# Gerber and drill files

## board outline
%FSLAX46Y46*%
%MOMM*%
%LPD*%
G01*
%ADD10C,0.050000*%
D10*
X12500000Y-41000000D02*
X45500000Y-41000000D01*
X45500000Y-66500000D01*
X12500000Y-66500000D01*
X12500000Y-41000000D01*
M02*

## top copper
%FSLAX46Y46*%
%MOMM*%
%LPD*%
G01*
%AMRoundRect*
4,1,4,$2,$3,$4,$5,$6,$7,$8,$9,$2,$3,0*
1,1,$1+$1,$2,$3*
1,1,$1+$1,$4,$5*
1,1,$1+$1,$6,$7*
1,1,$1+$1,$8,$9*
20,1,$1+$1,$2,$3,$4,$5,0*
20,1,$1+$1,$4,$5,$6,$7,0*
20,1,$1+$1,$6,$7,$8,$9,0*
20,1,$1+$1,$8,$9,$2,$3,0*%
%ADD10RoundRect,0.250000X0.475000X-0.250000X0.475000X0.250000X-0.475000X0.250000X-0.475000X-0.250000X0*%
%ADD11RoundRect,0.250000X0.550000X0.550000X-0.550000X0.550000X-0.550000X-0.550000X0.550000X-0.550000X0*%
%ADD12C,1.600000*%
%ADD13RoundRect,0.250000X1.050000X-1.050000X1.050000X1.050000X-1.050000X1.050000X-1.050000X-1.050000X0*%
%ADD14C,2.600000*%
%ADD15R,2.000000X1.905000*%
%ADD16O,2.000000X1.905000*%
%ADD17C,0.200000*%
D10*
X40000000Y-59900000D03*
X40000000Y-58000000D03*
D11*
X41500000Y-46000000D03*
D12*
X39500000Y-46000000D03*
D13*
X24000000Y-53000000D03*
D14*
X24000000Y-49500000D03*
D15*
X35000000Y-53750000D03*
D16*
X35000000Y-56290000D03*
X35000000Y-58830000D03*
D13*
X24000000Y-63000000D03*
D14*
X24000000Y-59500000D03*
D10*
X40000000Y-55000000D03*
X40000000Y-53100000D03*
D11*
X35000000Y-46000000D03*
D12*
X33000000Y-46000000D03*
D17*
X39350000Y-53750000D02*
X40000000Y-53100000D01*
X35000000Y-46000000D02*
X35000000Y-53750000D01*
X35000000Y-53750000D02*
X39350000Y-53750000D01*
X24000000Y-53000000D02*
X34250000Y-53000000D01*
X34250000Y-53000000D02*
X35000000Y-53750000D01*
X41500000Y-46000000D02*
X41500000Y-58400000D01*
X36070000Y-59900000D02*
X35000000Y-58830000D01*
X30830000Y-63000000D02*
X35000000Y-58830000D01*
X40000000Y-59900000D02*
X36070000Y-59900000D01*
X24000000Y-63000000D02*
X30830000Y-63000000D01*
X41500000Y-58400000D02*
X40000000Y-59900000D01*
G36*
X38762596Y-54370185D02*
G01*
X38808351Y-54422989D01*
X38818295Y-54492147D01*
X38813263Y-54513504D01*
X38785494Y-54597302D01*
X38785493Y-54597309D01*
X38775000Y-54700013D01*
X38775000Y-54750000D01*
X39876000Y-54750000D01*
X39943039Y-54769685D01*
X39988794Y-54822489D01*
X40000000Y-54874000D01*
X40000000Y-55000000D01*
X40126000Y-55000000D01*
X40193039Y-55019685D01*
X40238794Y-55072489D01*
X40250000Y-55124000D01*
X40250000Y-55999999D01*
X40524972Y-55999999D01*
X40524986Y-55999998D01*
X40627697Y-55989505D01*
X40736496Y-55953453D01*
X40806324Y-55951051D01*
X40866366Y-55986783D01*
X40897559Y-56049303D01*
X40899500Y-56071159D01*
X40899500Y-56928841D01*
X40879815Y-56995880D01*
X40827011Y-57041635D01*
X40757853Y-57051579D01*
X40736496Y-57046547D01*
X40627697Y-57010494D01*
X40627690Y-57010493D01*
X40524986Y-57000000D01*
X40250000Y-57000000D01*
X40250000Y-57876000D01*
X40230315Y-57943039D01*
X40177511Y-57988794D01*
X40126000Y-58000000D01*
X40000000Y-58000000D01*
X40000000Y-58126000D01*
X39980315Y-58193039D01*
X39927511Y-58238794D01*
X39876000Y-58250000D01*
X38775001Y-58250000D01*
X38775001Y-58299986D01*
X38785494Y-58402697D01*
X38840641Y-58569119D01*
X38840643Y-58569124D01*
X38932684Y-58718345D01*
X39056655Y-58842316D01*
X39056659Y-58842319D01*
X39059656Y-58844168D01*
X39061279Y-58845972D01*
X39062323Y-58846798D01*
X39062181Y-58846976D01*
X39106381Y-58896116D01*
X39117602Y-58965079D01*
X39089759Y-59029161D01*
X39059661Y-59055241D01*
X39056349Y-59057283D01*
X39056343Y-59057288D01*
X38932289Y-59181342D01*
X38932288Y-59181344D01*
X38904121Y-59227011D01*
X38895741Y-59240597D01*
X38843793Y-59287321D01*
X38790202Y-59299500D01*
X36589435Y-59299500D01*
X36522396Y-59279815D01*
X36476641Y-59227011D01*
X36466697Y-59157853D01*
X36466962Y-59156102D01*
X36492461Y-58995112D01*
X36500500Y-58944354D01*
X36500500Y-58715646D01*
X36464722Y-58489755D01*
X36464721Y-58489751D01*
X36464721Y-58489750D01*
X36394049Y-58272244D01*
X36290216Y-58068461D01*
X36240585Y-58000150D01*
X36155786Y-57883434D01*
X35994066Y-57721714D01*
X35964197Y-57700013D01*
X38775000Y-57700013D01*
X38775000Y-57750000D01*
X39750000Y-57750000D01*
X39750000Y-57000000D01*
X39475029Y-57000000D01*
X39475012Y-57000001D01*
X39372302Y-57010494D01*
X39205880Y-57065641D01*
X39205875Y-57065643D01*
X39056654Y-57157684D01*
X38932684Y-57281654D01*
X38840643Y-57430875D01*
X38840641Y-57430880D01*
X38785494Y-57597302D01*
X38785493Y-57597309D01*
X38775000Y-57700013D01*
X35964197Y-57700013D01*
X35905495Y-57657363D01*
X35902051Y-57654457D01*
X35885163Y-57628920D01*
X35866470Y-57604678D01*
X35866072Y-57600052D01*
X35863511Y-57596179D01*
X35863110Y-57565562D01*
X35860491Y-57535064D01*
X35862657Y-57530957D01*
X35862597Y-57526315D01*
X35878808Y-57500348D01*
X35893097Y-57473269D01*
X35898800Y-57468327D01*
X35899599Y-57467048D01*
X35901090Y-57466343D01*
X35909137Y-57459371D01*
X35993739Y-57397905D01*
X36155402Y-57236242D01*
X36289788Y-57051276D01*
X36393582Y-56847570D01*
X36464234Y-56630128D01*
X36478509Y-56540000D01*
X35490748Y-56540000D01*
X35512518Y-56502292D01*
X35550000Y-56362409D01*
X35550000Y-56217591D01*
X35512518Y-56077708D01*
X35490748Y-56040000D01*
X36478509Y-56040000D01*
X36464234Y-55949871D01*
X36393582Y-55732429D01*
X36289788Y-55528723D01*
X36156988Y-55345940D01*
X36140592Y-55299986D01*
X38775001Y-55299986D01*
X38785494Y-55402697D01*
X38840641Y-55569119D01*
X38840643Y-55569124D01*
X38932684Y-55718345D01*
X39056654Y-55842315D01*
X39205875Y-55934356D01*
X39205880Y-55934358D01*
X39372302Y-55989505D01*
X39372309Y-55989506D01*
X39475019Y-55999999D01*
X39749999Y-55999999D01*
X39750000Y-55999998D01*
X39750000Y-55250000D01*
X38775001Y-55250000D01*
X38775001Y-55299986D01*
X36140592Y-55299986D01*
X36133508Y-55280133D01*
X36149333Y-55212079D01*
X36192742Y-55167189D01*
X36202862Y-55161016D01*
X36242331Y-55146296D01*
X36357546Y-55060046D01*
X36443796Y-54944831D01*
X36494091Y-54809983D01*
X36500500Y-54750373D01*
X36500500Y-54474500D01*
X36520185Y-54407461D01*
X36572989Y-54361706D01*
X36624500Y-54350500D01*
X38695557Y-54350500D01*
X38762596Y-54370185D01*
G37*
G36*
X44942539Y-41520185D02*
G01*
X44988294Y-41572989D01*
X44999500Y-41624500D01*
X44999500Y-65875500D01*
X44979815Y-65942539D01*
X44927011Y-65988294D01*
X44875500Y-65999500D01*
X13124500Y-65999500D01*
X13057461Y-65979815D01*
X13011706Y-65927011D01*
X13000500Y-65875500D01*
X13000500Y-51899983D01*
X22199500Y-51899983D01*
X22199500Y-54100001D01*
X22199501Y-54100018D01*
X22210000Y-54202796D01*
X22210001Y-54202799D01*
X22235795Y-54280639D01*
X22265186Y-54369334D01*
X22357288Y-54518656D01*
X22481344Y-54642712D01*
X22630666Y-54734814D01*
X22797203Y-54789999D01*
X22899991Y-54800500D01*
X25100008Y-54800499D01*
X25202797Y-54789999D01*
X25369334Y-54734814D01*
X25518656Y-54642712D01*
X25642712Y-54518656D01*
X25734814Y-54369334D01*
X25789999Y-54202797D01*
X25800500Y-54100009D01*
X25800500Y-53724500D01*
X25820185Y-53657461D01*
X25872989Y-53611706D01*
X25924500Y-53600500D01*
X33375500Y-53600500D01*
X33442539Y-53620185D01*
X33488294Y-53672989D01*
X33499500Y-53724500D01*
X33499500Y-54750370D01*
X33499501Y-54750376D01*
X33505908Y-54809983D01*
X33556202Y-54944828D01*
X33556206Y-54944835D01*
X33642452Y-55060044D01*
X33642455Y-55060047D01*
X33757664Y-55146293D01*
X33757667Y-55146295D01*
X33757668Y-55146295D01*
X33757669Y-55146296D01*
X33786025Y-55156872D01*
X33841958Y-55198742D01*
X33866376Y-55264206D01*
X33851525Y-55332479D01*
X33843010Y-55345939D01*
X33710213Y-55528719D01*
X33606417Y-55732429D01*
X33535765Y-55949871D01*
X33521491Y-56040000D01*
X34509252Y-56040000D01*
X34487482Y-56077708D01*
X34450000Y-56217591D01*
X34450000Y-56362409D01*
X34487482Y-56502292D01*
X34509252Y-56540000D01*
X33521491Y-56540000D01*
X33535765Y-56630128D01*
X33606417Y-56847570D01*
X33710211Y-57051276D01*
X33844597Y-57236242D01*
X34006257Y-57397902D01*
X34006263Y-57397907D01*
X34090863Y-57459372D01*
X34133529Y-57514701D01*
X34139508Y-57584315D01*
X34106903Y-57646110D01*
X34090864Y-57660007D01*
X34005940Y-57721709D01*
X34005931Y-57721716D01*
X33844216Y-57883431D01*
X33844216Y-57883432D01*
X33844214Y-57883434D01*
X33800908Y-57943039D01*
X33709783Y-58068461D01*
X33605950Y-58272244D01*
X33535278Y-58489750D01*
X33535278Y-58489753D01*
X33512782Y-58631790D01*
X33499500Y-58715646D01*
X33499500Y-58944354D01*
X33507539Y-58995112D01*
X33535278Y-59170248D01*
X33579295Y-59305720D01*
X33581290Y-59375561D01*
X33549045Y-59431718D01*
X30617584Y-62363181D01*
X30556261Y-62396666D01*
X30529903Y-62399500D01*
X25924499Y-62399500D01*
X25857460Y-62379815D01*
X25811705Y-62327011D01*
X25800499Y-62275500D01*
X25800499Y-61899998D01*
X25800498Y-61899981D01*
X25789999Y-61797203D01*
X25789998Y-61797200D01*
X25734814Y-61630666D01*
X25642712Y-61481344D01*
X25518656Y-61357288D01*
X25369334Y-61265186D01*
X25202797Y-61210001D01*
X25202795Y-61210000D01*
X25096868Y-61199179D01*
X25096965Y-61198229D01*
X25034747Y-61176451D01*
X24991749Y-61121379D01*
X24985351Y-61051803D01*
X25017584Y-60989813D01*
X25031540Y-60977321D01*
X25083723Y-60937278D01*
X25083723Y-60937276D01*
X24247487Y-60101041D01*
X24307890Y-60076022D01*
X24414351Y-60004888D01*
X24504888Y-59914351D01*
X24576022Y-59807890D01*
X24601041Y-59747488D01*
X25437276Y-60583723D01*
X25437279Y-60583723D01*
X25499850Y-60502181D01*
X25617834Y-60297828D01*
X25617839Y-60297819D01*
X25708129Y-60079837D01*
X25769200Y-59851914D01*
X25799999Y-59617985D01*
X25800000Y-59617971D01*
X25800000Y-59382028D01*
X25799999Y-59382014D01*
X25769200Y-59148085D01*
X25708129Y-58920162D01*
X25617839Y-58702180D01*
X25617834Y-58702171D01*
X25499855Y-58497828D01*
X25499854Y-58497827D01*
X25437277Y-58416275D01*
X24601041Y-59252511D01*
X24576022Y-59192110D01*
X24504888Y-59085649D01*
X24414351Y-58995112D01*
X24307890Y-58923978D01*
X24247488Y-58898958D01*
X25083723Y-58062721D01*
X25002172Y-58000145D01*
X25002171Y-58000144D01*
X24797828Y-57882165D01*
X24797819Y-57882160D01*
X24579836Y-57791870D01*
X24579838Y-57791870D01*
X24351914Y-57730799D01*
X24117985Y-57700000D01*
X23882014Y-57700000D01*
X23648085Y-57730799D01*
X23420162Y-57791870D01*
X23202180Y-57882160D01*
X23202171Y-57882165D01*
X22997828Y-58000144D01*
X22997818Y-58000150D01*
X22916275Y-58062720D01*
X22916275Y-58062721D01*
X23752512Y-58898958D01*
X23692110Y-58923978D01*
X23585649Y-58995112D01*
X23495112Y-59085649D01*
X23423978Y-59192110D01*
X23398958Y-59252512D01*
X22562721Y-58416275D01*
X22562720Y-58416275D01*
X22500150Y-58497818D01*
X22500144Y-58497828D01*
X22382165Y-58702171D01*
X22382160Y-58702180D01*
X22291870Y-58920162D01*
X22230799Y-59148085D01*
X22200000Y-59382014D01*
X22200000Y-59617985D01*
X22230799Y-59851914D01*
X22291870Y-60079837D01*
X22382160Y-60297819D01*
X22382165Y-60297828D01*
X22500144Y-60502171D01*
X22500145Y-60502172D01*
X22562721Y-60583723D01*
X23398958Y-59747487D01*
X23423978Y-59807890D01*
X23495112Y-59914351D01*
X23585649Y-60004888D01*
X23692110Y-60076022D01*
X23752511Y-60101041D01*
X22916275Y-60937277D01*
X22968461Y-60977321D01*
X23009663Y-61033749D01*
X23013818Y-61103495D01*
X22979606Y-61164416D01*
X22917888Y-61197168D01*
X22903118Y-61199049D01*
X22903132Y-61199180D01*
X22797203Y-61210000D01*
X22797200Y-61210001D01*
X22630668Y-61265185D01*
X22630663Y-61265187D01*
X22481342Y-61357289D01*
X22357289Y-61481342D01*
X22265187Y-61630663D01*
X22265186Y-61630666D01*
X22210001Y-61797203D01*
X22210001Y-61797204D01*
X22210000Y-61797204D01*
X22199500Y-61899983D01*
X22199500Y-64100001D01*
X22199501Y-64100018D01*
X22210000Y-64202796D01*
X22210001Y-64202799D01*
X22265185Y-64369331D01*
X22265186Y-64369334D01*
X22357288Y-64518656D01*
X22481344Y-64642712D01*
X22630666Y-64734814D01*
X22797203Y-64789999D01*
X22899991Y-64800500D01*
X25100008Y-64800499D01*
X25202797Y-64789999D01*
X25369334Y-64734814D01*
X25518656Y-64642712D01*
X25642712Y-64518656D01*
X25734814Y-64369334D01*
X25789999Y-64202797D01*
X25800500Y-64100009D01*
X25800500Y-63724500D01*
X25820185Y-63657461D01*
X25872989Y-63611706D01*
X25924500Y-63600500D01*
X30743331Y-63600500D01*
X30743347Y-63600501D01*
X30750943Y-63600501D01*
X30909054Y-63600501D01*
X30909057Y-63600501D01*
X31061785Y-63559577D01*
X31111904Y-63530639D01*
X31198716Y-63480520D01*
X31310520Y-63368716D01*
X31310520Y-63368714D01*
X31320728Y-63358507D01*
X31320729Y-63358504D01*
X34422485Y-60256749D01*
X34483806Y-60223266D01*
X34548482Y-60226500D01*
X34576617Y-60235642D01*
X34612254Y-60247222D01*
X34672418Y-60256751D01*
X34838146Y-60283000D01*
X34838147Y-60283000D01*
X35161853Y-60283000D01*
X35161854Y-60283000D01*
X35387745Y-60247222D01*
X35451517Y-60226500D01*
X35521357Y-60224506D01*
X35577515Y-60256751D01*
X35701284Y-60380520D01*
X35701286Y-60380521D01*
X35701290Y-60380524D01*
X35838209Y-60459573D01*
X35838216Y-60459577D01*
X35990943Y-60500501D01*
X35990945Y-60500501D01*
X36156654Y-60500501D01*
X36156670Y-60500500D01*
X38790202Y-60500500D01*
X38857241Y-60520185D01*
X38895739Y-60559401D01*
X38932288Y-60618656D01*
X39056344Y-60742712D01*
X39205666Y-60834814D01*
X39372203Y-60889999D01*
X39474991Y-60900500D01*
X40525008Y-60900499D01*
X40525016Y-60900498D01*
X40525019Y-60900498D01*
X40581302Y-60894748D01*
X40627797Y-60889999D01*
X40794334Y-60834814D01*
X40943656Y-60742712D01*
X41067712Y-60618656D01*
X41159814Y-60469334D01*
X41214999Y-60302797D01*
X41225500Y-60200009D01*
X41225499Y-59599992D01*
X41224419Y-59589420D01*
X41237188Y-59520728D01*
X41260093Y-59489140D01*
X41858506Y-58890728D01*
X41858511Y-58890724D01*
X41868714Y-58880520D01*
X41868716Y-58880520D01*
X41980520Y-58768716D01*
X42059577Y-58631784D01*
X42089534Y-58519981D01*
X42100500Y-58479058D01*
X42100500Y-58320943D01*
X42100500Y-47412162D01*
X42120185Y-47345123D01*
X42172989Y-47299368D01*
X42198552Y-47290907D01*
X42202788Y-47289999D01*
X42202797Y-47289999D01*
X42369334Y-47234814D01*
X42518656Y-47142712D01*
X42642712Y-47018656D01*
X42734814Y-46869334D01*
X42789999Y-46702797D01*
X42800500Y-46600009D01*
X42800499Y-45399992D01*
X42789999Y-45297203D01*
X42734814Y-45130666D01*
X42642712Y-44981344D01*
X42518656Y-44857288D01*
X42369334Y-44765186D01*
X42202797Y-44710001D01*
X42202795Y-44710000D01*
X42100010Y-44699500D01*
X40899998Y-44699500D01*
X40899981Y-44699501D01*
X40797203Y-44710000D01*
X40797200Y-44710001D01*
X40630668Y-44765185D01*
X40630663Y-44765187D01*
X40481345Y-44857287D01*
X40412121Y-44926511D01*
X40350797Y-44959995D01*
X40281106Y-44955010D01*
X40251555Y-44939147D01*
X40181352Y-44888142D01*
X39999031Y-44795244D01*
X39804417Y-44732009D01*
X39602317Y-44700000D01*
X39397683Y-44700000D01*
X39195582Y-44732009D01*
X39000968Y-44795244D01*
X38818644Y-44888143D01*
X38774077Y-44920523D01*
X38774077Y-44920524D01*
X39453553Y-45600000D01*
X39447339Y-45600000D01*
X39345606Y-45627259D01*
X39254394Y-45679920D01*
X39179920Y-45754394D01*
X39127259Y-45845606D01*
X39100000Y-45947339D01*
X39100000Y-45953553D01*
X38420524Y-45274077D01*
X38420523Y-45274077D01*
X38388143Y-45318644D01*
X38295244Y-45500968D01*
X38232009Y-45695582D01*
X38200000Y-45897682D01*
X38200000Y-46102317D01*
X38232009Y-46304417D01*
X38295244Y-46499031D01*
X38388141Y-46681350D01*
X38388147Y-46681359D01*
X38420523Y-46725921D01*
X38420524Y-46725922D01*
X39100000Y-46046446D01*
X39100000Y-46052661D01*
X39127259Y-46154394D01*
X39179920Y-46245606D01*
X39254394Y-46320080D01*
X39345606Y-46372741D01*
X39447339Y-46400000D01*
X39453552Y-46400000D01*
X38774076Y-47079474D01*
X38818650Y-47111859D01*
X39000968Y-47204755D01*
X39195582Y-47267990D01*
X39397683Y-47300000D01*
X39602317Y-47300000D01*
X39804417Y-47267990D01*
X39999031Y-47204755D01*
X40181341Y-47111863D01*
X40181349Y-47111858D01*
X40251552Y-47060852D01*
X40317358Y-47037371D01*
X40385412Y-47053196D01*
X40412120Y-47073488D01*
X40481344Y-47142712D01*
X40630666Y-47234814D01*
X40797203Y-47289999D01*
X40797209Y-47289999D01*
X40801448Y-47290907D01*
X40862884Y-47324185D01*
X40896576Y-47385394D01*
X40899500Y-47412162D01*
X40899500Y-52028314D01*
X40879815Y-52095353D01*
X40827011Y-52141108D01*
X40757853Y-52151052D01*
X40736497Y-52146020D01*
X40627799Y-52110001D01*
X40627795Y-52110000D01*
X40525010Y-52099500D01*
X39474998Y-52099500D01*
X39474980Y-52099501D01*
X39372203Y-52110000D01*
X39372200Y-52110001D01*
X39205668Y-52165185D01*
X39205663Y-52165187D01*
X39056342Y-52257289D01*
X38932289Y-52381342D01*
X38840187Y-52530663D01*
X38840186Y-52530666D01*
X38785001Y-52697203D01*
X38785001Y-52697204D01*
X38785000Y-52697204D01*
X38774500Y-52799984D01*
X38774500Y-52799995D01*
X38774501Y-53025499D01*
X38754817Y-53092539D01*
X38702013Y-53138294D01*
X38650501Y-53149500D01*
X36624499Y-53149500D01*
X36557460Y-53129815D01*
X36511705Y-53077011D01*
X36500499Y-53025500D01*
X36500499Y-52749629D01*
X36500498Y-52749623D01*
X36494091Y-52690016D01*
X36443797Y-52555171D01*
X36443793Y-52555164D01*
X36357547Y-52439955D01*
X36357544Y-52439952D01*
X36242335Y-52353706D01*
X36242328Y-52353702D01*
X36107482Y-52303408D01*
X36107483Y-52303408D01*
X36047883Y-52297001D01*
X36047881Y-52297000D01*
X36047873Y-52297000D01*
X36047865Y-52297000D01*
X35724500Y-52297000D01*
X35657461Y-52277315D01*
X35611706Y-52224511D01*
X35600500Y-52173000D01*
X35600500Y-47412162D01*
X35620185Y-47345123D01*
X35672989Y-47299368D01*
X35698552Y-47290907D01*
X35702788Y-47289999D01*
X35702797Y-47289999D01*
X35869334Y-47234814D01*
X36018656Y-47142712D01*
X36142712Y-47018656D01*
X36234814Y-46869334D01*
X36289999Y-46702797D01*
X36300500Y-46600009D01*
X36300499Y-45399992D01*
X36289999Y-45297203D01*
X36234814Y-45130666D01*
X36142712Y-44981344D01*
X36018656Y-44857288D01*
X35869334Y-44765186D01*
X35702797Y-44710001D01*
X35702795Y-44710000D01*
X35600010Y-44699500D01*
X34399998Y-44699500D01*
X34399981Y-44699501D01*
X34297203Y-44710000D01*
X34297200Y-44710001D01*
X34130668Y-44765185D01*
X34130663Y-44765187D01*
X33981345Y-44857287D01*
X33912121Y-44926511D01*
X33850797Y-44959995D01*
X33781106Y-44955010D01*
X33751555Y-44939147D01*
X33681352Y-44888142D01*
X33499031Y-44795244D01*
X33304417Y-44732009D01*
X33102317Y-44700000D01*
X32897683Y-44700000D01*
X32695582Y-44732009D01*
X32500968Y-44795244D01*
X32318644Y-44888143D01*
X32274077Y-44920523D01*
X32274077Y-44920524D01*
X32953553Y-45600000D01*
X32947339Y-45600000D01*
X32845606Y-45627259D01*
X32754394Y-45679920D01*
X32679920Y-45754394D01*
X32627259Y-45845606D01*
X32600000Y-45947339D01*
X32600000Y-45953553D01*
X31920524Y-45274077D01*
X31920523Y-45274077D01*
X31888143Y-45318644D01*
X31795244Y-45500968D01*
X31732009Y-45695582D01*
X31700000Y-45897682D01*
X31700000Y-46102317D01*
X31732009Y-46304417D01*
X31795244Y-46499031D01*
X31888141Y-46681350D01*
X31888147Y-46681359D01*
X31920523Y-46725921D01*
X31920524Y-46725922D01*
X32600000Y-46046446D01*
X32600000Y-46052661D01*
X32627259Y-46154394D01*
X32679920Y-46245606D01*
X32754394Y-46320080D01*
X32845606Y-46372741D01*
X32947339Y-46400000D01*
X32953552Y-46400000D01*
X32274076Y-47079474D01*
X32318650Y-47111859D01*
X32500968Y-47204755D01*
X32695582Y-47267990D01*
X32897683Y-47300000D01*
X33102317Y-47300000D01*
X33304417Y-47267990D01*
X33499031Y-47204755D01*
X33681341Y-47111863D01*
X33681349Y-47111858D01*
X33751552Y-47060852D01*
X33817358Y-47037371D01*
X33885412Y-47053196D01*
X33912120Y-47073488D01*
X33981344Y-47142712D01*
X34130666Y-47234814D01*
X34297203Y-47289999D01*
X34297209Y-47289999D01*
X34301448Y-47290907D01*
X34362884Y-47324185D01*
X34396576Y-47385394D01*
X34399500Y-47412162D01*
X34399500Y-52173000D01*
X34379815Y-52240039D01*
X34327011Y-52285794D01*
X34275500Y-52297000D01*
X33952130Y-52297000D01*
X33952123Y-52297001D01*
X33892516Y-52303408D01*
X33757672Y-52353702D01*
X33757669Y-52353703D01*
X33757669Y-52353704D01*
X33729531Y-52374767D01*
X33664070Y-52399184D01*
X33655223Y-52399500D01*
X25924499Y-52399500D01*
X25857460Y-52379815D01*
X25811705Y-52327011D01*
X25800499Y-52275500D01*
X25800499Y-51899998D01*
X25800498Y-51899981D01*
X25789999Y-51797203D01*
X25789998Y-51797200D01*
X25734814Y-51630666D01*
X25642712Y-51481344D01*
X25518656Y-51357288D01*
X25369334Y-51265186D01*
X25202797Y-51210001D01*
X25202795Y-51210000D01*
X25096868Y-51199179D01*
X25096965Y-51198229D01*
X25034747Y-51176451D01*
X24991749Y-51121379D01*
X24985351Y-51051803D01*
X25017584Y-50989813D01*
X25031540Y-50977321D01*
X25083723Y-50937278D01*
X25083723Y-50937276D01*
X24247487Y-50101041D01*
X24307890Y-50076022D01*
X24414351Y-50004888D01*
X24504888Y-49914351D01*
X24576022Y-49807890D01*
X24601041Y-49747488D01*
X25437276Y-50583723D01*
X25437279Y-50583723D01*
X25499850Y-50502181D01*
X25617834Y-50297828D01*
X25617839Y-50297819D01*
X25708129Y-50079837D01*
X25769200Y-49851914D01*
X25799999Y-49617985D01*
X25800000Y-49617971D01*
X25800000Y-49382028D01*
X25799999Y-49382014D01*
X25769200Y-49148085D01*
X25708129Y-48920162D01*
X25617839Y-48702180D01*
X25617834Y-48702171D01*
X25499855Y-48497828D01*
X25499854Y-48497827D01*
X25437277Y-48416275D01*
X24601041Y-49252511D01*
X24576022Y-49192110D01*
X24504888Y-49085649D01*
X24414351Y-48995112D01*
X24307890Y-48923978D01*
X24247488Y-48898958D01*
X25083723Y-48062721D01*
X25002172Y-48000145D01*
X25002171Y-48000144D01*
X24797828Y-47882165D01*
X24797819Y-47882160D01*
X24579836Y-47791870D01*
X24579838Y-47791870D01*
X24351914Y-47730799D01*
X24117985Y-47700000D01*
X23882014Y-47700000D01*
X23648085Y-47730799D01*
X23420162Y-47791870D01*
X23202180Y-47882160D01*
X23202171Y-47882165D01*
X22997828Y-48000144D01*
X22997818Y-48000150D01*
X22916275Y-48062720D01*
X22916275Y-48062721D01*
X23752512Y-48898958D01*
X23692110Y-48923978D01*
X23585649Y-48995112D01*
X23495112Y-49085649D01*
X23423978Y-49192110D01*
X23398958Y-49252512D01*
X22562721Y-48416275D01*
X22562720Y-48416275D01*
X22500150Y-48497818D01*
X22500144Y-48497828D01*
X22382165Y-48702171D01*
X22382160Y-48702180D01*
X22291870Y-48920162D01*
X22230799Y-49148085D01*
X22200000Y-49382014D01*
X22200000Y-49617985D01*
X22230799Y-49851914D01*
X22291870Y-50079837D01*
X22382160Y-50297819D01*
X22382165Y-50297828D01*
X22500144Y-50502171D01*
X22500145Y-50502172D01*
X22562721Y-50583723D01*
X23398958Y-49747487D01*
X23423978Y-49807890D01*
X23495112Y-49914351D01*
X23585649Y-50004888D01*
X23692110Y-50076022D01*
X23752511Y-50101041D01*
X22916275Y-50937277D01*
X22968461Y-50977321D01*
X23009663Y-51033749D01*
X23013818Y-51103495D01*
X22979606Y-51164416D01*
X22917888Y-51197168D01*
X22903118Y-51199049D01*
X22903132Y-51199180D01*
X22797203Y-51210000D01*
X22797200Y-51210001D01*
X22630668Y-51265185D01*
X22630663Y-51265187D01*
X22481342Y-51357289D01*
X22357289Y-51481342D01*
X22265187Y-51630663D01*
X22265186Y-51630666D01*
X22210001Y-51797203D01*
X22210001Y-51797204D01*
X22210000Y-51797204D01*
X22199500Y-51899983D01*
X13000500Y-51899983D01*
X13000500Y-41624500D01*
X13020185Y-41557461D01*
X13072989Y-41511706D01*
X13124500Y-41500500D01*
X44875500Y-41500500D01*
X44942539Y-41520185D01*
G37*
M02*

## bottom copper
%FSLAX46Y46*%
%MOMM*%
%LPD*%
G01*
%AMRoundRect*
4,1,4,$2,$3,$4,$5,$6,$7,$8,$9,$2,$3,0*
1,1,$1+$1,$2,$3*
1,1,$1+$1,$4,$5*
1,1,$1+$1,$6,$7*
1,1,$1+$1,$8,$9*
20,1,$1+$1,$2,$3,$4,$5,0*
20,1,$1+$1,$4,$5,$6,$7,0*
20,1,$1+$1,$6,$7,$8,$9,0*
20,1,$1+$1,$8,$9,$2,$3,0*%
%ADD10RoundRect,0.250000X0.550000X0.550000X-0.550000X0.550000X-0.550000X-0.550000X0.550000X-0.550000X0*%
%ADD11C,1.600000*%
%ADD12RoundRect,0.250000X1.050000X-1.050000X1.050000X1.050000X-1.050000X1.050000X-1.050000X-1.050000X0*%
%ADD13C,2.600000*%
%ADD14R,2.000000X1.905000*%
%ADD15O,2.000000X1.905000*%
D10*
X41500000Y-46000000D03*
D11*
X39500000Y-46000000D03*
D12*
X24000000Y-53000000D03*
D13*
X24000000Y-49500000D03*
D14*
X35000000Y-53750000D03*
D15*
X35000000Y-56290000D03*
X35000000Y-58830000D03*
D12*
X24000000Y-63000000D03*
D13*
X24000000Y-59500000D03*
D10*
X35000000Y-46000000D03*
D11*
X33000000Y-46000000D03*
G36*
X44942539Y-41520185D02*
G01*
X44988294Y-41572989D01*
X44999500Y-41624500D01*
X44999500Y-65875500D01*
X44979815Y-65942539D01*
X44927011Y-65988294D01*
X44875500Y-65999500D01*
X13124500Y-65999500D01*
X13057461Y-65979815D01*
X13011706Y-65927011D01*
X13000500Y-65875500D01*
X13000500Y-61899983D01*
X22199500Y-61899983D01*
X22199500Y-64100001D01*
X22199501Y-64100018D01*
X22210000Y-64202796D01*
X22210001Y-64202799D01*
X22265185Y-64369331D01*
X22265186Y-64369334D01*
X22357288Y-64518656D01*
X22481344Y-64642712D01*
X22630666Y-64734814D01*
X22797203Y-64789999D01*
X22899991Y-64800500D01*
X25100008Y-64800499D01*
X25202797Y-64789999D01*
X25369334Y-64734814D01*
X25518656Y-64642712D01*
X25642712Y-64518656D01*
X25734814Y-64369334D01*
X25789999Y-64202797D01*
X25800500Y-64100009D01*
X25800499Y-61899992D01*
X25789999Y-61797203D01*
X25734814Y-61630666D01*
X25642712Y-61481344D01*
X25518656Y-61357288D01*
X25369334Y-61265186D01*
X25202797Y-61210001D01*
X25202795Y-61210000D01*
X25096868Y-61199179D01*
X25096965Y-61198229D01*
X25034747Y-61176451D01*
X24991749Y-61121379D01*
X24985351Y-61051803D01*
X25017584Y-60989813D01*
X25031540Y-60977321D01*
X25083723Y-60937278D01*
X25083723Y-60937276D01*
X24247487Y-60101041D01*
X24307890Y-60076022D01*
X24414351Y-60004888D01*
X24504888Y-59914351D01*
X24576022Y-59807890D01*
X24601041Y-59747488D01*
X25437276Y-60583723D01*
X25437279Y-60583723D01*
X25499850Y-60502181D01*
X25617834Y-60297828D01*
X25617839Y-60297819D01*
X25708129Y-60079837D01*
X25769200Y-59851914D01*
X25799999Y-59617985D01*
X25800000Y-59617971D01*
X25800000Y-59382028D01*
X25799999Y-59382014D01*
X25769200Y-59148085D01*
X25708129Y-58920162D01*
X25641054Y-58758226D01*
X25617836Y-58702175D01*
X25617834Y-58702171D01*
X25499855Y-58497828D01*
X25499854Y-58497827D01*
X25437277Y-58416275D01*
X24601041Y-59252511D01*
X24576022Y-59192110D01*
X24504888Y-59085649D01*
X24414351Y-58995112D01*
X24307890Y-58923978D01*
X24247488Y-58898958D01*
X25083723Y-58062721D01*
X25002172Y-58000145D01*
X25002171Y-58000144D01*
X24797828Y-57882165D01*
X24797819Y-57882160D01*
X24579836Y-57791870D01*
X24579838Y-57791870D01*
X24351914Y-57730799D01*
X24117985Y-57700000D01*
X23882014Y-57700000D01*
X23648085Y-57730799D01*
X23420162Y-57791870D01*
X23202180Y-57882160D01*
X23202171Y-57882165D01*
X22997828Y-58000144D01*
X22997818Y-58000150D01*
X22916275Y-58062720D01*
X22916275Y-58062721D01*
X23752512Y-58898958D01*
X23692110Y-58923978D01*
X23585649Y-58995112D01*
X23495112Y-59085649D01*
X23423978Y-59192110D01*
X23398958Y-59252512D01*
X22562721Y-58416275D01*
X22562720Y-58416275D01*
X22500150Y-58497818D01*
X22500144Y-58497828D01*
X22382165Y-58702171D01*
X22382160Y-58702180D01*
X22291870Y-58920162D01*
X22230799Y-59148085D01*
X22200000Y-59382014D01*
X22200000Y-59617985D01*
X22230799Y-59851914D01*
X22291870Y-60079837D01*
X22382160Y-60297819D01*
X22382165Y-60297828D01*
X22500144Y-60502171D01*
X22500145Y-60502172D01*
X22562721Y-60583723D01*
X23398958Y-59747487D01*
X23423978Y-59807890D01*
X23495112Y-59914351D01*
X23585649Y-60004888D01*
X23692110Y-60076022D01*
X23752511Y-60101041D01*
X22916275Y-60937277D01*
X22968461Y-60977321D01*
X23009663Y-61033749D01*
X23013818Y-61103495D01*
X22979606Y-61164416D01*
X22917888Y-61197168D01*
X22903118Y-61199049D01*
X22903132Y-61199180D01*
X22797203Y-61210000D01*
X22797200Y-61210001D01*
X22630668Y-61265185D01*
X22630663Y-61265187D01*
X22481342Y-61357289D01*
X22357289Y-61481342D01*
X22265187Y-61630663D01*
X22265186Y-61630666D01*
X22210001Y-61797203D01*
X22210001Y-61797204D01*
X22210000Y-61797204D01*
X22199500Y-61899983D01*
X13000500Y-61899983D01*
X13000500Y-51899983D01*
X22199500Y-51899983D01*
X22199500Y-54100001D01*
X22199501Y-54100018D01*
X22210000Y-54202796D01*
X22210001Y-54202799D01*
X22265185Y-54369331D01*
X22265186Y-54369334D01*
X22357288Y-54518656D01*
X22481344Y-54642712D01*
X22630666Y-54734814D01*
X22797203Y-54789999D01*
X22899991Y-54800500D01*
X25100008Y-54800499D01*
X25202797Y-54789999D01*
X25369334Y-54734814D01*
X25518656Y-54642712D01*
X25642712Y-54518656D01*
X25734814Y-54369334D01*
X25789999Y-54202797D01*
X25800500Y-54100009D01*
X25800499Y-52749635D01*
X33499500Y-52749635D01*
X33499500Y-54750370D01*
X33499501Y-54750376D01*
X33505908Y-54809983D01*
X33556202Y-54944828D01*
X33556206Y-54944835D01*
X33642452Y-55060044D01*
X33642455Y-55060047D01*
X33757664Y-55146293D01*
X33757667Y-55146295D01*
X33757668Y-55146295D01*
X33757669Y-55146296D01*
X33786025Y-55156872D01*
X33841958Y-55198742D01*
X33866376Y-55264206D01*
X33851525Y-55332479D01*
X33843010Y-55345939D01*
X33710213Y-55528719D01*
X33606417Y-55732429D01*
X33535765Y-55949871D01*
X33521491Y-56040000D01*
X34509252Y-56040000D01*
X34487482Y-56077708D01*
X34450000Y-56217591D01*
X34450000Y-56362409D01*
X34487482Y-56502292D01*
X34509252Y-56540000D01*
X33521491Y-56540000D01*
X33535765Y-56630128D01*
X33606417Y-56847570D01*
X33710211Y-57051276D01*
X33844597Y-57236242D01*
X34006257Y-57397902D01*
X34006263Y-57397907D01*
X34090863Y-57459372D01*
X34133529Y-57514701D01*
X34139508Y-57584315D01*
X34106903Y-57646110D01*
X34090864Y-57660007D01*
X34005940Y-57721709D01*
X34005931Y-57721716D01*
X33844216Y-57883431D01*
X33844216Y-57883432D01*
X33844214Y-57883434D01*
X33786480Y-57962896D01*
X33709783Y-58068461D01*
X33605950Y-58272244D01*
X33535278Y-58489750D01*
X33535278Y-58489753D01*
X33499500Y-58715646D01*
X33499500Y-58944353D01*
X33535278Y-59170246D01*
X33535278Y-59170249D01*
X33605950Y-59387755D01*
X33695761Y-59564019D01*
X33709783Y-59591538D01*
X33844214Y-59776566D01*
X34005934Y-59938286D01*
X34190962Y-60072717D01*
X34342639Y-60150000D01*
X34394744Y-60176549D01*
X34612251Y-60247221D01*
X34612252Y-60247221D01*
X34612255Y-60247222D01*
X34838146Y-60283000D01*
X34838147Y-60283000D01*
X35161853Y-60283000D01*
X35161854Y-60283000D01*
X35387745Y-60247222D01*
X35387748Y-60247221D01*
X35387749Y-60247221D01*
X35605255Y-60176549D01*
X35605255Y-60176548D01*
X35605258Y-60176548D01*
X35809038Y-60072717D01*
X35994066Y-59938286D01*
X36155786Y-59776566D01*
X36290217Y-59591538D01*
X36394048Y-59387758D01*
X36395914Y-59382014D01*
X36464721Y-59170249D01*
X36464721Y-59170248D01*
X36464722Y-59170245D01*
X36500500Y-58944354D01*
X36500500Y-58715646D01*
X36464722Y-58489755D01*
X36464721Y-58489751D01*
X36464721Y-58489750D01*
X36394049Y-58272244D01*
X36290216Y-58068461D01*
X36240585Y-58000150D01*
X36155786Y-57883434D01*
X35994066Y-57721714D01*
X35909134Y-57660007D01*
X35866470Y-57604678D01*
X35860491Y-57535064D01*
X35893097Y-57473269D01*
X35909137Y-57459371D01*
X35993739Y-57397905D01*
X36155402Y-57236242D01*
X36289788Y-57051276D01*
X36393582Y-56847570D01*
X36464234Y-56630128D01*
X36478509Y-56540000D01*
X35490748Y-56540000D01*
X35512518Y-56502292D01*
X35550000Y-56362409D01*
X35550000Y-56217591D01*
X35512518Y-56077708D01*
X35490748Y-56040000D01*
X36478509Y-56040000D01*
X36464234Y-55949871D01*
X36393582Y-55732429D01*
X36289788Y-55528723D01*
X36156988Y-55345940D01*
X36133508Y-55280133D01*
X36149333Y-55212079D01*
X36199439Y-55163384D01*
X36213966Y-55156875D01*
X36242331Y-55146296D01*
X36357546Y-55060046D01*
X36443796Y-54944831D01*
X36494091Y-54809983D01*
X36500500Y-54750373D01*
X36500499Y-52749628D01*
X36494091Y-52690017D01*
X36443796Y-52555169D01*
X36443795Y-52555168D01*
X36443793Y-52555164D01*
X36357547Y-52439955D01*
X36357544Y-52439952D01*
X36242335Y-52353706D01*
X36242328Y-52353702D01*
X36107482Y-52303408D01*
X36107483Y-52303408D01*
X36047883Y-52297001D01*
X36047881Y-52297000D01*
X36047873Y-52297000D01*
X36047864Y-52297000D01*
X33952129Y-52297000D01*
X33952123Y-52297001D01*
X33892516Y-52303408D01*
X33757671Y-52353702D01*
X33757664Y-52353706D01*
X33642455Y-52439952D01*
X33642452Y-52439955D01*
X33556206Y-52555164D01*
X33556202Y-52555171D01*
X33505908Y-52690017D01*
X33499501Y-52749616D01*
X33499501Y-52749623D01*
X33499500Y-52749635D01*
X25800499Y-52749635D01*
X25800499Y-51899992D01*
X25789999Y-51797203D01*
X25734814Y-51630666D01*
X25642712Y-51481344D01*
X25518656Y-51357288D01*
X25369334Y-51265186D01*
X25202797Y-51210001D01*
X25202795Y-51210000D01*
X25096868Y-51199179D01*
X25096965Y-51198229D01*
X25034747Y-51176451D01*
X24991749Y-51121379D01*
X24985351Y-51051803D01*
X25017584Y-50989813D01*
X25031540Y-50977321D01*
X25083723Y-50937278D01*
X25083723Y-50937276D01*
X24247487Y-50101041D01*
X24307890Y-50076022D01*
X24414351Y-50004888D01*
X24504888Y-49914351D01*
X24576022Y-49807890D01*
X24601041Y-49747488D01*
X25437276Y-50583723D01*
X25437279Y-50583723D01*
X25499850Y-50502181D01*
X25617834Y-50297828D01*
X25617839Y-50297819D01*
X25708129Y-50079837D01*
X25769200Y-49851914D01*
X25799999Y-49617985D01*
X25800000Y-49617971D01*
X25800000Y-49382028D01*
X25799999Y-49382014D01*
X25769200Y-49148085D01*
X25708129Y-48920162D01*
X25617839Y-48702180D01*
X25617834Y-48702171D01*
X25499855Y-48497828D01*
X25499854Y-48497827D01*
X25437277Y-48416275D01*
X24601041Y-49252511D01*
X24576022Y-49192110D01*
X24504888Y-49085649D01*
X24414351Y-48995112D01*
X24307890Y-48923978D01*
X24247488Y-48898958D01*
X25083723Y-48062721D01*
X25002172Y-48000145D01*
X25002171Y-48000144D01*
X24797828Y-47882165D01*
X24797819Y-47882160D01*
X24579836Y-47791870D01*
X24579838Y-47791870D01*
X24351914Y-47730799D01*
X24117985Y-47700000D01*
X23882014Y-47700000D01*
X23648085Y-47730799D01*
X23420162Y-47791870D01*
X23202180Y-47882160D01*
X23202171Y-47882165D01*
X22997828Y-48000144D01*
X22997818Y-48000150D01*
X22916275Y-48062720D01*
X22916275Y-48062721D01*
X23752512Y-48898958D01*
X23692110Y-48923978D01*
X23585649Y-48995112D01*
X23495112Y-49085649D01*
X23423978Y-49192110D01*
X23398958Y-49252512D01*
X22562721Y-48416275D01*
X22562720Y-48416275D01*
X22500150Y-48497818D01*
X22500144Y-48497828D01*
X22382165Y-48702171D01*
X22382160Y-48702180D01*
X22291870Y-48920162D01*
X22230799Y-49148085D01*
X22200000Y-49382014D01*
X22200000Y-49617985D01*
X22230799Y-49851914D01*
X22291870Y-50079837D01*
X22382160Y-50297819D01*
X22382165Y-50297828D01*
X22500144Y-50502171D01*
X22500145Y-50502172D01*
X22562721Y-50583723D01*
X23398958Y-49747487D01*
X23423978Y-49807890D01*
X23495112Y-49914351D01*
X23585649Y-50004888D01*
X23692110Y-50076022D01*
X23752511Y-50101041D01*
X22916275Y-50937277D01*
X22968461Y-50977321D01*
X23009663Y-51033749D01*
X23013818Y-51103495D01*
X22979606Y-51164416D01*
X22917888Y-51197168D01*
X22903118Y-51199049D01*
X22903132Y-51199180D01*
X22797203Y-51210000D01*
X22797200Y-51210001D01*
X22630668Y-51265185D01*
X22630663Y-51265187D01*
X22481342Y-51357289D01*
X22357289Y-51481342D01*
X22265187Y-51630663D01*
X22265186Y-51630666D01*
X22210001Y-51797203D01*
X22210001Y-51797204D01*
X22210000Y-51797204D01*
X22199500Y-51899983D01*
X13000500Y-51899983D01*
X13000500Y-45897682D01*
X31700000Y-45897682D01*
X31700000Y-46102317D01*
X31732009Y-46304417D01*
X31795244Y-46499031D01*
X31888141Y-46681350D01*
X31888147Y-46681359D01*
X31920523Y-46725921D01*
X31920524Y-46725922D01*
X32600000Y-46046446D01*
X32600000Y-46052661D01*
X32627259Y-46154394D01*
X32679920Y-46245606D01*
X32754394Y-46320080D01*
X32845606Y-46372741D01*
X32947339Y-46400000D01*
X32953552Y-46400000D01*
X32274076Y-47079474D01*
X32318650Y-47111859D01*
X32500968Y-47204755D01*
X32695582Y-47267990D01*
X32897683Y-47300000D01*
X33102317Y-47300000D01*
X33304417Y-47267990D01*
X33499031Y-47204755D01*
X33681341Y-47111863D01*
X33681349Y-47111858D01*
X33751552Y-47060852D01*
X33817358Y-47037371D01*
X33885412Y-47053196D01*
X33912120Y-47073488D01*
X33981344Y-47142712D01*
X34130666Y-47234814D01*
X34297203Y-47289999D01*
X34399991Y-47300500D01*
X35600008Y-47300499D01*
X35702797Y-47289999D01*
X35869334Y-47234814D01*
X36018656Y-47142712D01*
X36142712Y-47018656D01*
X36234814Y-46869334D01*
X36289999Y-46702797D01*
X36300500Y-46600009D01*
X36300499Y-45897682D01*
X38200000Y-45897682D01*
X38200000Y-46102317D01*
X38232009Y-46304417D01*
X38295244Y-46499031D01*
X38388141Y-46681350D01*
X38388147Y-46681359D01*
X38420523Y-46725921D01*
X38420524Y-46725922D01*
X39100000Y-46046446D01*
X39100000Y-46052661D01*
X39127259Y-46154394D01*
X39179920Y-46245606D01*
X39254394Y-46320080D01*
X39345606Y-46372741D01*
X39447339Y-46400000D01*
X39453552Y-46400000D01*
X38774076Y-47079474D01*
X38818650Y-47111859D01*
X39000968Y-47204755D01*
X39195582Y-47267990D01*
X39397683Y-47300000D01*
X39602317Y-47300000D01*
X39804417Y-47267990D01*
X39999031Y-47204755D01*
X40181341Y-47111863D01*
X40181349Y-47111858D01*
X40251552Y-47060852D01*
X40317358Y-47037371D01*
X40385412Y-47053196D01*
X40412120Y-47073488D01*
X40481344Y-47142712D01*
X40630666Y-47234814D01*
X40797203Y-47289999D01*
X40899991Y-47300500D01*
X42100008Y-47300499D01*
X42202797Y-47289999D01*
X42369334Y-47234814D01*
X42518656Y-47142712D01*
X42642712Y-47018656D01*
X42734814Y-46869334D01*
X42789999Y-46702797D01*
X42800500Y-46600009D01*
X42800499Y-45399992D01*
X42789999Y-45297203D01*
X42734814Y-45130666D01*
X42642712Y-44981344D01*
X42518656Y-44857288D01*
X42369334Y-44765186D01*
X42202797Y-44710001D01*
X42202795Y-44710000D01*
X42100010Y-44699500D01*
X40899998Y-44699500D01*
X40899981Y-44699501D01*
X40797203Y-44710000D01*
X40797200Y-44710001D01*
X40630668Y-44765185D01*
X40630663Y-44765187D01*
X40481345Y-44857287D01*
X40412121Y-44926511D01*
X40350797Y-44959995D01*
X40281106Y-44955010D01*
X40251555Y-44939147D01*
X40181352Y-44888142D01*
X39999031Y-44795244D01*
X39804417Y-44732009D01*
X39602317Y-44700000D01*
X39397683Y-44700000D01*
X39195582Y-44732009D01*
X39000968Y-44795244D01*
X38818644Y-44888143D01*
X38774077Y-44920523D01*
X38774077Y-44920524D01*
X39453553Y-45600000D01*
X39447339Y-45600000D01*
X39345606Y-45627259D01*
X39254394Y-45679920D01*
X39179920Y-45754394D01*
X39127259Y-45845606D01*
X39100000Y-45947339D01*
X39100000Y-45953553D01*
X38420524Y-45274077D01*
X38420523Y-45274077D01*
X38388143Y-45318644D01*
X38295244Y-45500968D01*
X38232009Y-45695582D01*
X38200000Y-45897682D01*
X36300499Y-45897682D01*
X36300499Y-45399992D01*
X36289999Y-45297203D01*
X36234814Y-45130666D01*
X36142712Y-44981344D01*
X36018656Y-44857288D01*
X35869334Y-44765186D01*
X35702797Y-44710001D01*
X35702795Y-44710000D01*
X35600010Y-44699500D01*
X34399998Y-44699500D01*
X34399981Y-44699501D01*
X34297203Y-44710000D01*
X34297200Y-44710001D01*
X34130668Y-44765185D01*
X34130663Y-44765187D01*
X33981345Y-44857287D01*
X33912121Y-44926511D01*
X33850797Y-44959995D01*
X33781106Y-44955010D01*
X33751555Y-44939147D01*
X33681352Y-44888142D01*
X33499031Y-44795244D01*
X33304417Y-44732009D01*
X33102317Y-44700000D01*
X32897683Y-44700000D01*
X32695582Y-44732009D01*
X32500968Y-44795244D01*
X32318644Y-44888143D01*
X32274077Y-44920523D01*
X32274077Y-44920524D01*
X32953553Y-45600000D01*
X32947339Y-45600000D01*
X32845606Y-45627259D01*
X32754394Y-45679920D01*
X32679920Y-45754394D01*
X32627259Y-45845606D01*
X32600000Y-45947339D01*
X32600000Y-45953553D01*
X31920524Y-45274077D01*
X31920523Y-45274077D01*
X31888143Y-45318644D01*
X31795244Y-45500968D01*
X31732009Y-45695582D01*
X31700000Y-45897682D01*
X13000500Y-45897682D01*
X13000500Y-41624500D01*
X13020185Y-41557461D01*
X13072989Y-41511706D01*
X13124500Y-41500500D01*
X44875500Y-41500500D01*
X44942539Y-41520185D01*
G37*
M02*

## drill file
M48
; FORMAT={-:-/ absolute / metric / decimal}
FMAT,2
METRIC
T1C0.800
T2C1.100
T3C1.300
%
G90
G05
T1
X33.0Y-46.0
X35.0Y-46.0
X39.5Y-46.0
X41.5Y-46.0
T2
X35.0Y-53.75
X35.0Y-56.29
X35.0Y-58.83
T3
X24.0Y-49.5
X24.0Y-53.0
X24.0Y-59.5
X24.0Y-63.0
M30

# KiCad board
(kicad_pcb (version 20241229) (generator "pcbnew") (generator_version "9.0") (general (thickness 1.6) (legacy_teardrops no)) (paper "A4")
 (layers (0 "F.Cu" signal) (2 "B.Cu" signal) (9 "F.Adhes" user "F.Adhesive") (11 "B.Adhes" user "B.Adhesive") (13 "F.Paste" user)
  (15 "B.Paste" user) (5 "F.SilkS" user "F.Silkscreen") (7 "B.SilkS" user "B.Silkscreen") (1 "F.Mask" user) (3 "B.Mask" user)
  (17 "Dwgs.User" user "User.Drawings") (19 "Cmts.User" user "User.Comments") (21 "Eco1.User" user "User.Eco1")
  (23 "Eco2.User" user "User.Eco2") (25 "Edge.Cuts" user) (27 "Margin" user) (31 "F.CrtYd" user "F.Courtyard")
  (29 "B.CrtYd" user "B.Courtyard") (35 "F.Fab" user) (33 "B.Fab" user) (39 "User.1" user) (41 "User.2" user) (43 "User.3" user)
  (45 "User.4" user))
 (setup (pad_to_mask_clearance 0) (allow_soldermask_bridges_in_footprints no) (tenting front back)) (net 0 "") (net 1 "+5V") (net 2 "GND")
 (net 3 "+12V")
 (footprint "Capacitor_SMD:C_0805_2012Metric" (layer "F.Cu") (at 40 58.95 90)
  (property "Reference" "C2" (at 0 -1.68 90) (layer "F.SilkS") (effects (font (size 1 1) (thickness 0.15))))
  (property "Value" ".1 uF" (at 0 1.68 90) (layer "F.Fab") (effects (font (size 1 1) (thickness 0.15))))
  (pad "1" smd roundrect (at -0.95 0 90) (size 1 1.45) (layers "F.Cu" "F.Mask" "F.Paste") (roundrect_rratio 0.25) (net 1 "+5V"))
  (pad "2" smd roundrect (at 0.95 0 90) (size 1 1.45) (layers "F.Cu" "F.Mask" "F.Paste") (roundrect_rratio 0.25) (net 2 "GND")))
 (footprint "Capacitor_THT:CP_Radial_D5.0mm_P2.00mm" (layer "F.Cu") (at 41.5 46 180)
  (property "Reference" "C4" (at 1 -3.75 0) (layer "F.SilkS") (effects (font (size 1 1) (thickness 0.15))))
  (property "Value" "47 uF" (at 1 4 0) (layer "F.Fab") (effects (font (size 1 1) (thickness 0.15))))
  (pad "1" thru_hole roundrect (at 0 0 180) (size 1.6 1.6) (drill 0.8) (layers "*.Cu" "*.Mask") (remove_unused_layers no)
   (roundrect_rratio 0.15625) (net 1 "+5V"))
  (pad "2" thru_hole circle (at 2 0 180) (size 1.6 1.6) (drill 0.8) (layers "*.Cu" "*.Mask") (remove_unused_layers no) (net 2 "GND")))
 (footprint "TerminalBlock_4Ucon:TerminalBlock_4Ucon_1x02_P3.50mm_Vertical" (layer "F.Cu") (at 24 53 90)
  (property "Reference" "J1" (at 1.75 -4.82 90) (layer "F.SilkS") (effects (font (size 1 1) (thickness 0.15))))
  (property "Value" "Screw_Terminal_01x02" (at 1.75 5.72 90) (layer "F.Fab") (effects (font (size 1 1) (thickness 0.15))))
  (pad "1" thru_hole roundrect (at 0 0 90) (size 2.6 2.6) (drill 1.3) (layers "*.Cu" "*.Mask") (remove_unused_layers no)
   (roundrect_rratio 0.096154) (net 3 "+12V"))
  (pad "2" thru_hole circle (at 3.5 0 90) (size 2.6 2.6) (drill 1.3) (layers "*.Cu" "*.Mask") (remove_unused_layers no) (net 2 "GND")))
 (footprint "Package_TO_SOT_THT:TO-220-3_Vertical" (layer "F.Cu") (at 35 53.75 -90)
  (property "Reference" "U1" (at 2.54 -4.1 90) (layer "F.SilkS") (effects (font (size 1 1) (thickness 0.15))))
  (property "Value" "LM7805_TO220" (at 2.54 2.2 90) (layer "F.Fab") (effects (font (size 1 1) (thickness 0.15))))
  (pad "1" thru_hole rect (at 0 0 270) (size 1.905 2) (drill 1.1) (layers "*.Cu" "*.Mask") (remove_unused_layers no) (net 3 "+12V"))
  (pad "2" thru_hole oval (at 2.54 0 270) (size 1.905 2) (drill 1.1) (layers "*.Cu" "*.Mask") (remove_unused_layers no) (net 2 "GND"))
  (pad "3" thru_hole oval (at 5.08 0 270) (size 1.905 2) (drill 1.1) (layers "*.Cu" "*.Mask") (remove_unused_layers no) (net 1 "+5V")))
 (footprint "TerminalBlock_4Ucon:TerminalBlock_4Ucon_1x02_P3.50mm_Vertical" (layer "F.Cu") (at 24 63 90)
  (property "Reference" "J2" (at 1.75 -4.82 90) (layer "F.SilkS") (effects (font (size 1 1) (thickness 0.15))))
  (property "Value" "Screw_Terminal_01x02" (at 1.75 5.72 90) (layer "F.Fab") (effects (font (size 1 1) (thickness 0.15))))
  (pad "1" thru_hole roundrect (at 0 0 90) (size 2.6 2.6) (drill 1.3) (layers "*.Cu" "*.Mask") (remove_unused_layers no)
   (roundrect_rratio 0.096154) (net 1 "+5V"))
  (pad "2" thru_hole circle (at 3.5 0 90) (size 2.6 2.6) (drill 1.3) (layers "*.Cu" "*.Mask") (remove_unused_layers no) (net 2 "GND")))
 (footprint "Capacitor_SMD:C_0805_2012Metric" (layer "F.Cu") (at 40 54.05 90)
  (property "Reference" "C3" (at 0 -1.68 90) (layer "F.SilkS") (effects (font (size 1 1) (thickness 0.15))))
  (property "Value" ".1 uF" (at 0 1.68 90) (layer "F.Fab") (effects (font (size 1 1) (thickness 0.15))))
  (pad "1" smd roundrect (at -0.95 0 90) (size 1 1.45) (layers "F.Cu" "F.Mask" "F.Paste") (roundrect_rratio 0.25) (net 2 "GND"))
  (pad "2" smd roundrect (at 0.95 0 90) (size 1 1.45) (layers "F.Cu" "F.Mask" "F.Paste") (roundrect_rratio 0.25) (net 3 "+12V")))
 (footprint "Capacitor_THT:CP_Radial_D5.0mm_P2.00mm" (layer "F.Cu") (at 35 46 180)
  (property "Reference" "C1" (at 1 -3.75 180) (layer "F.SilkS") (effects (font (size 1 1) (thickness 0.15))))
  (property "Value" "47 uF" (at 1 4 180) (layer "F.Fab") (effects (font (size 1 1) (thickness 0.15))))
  (pad "1" thru_hole roundrect (at 0 0 180) (size 1.6 1.6) (drill 0.8) (layers "*.Cu" "*.Mask") (remove_unused_layers no)
   (roundrect_rratio 0.15625) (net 3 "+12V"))
  (pad "2" thru_hole circle (at 2 0 180) (size 1.6 1.6) (drill 0.8) (layers "*.Cu" "*.Mask") (remove_unused_layers no) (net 2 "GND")))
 (gr_rect (start 12.5 41) (end 45.5 66.5) (stroke (width 0.05) (type default)) (fill no) (layer "Edge.Cuts"))
 (segment (start 39.35 53.75) (end 40 53.1) (width 0.2) (layer "F.Cu") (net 3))
 (segment (start 35 46) (end 35 53.75) (width 0.2) (layer "F.Cu") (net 3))
 (segment (start 35 53.75) (end 39.35 53.75) (width 0.2) (layer "F.Cu") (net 3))
 (segment (start 24 53) (end 34.25 53) (width 0.2) (layer "F.Cu") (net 3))
 (segment (start 34.25 53) (end 35 53.75) (width 0.2) (layer "F.Cu") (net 3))
 (segment (start 41.5 46) (end 41.5 58.4) (width 0.2) (layer "F.Cu") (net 1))
 (segment (start 36.07 59.9) (end 35 58.83) (width 0.2) (layer "F.Cu") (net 1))
 (segment (start 30.83 63) (end 35 58.83) (width 0.2) (layer "F.Cu") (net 1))
 (segment (start 40 59.9) (end 36.07 59.9) (width 0.2) (layer "F.Cu") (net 1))
 (segment (start 24 63) (end 30.83 63) (width 0.2) (layer "F.Cu") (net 1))
 (segment (start 41.5 58.4) (end 40 59.9) (width 0.2) (layer "F.Cu") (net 1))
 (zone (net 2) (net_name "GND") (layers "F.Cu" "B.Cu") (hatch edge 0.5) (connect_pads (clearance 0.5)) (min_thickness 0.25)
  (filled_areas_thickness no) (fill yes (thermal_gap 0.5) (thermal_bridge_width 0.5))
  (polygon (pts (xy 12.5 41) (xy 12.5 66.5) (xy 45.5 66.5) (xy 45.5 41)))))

